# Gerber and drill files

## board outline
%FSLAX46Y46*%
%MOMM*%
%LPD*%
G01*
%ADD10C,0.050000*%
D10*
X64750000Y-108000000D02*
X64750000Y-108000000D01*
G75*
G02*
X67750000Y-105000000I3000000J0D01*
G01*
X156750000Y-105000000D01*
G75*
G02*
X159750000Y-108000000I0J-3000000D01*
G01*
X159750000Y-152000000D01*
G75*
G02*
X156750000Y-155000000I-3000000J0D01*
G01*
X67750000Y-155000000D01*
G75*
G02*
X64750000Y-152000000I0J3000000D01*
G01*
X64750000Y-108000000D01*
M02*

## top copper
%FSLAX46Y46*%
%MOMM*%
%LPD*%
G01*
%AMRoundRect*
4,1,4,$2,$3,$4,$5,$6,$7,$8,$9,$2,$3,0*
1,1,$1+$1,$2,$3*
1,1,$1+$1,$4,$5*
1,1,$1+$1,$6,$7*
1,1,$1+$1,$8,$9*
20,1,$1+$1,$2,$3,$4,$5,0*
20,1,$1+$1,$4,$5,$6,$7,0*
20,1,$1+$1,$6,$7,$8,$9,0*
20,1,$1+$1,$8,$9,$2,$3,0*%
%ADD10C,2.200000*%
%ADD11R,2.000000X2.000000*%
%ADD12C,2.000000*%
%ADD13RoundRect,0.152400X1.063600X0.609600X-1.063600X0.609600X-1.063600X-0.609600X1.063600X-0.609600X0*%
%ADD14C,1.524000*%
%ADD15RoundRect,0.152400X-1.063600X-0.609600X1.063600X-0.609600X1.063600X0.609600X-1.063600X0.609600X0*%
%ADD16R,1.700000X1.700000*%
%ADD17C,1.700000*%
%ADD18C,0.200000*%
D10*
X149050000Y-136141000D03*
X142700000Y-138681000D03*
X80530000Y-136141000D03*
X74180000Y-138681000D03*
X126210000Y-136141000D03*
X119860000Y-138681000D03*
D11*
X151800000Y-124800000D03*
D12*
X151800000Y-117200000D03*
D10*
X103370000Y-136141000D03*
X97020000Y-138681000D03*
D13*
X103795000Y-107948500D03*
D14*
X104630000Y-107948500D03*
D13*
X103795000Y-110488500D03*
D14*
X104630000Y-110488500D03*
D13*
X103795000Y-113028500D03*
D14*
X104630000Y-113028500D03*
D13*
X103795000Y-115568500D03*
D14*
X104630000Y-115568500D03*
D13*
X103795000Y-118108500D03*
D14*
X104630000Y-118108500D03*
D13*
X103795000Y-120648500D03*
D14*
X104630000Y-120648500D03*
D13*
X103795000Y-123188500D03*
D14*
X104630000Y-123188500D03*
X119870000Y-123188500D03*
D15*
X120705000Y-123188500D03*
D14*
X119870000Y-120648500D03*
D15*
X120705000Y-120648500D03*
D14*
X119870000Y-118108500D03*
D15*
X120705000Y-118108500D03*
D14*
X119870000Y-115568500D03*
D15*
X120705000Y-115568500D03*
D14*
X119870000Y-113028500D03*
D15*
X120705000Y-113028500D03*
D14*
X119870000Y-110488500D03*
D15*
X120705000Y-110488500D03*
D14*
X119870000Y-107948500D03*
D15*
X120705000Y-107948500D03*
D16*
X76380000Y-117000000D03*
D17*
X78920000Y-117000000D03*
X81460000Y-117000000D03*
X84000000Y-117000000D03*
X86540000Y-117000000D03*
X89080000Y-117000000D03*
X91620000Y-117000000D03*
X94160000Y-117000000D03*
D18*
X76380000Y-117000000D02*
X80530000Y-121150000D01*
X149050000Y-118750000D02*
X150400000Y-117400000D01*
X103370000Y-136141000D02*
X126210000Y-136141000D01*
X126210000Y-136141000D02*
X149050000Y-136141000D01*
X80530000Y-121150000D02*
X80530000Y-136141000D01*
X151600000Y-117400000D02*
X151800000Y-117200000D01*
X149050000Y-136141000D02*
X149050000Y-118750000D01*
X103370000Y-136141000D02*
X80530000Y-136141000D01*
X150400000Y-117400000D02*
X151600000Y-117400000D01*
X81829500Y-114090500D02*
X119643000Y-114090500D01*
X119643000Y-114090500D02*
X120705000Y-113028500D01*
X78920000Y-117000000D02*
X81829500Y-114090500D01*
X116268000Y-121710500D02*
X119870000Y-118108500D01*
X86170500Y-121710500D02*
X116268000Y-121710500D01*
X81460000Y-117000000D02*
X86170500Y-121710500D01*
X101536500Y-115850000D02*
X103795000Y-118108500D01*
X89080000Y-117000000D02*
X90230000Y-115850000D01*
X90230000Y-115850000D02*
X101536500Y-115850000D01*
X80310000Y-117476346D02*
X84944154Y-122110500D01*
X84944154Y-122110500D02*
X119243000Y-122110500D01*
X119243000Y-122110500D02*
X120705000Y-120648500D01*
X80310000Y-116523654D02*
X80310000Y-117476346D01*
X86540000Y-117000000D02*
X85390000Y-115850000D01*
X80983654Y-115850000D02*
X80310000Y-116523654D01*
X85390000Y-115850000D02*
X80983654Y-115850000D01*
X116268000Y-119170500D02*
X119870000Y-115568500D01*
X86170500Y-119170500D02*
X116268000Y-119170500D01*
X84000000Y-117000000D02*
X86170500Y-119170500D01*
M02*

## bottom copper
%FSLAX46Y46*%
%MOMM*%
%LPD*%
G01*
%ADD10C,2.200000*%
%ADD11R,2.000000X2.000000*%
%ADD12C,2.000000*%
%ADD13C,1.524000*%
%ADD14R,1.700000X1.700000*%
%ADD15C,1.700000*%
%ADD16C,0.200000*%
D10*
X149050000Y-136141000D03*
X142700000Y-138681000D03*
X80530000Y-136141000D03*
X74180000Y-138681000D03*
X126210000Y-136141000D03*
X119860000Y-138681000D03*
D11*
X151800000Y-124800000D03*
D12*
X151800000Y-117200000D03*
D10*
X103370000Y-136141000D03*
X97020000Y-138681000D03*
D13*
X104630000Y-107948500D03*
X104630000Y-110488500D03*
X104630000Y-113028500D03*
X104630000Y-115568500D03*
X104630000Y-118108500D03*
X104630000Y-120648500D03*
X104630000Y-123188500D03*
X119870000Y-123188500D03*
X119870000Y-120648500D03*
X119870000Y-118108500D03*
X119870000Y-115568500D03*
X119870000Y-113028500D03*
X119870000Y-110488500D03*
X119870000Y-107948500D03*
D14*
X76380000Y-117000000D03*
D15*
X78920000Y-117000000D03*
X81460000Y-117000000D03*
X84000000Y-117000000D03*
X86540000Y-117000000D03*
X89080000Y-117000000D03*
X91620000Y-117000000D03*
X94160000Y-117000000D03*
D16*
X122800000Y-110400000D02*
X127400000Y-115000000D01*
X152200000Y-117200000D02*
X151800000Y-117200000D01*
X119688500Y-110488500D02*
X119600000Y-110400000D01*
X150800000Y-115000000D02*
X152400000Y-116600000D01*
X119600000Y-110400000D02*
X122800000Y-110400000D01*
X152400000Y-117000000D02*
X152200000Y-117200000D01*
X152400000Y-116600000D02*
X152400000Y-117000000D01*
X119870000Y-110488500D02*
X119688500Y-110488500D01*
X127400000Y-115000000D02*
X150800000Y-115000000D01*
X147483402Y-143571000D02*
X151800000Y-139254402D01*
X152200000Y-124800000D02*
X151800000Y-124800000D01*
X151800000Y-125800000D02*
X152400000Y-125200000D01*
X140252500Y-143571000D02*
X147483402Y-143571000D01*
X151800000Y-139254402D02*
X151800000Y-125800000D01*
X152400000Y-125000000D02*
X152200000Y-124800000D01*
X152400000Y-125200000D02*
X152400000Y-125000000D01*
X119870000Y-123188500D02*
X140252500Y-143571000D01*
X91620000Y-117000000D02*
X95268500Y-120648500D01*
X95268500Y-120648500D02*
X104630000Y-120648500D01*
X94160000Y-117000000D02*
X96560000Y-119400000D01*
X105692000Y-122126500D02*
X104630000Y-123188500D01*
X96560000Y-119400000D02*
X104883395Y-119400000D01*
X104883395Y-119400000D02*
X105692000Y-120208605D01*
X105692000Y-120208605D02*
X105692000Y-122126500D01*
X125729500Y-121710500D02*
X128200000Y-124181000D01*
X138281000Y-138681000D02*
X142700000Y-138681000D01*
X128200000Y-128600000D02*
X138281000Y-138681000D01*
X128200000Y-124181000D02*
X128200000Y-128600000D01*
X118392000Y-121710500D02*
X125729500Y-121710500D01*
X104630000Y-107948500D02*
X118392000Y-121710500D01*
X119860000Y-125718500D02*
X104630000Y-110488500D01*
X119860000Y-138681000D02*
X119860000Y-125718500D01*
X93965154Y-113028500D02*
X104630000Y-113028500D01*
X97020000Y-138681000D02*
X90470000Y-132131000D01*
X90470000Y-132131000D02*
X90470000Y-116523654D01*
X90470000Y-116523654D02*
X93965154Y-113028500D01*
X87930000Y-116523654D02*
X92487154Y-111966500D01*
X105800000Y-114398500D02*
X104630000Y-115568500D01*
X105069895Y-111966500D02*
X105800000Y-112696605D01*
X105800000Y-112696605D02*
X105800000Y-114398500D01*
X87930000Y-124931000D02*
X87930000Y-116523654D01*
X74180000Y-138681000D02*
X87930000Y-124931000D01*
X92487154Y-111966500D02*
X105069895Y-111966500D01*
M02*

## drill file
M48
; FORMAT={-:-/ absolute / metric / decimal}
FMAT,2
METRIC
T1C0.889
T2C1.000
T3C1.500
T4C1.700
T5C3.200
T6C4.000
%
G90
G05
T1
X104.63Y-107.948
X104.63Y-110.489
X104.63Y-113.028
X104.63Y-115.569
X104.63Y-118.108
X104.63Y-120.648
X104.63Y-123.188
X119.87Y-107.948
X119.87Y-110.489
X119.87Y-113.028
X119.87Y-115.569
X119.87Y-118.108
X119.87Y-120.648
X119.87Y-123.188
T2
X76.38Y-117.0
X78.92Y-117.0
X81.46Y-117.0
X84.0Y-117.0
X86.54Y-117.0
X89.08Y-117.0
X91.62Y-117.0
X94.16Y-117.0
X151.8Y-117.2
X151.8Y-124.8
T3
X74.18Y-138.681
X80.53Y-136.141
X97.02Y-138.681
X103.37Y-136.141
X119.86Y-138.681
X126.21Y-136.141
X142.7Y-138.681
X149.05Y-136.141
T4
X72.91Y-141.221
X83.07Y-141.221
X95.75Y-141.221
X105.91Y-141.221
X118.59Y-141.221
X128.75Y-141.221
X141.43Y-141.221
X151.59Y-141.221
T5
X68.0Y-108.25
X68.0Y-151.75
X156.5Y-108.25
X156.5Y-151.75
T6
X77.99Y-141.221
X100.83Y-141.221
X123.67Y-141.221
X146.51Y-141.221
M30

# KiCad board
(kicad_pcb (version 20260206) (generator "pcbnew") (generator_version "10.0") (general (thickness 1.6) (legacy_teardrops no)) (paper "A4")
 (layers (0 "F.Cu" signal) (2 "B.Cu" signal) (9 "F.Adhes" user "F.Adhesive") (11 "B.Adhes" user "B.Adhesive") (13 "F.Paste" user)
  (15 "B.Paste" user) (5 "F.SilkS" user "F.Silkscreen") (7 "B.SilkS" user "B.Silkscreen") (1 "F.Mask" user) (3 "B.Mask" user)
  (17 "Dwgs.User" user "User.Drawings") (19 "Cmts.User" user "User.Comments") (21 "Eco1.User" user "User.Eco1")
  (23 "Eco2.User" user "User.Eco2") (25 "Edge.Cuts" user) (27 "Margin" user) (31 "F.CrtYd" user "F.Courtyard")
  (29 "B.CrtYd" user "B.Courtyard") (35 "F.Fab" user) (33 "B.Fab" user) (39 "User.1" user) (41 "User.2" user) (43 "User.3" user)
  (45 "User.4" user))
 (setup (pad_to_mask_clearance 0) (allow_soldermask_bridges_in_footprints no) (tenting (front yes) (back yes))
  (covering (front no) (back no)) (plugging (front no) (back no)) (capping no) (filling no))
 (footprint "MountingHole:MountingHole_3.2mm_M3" (layer "F.Cu") (at 156.5 108.25 90)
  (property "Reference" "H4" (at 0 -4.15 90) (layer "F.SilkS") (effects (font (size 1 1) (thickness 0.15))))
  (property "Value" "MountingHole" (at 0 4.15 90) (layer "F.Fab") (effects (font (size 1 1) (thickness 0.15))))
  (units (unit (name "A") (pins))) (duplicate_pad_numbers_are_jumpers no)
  (pad "" np_thru_hole circle (at 0 0 90) (size 3.2 3.2) (drill 3.2) (layers "*.Cu" "*.Mask")))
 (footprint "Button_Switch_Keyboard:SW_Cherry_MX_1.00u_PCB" (layer "F.Cu") (at 149.05 136.141)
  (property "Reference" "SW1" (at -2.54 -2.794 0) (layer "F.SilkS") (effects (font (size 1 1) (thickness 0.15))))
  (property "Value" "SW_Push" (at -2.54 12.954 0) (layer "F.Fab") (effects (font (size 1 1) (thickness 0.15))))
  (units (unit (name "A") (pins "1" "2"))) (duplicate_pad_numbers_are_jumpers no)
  (pad "" np_thru_hole circle (at -7.62 5.08) (size 1.7 1.7) (drill 1.7) (layers "*.Cu" "*.Mask"))
  (pad "" np_thru_hole circle (at -2.54 5.08) (size 4 4) (drill 4) (layers "*.Cu" "*.Mask"))
  (pad "" np_thru_hole circle (at 2.54 5.08) (size 1.7 1.7) (drill 1.7) (layers "*.Cu" "*.Mask"))
  (pad "1" thru_hole circle (at 0 0) (size 2.2 2.2) (drill 1.5) (layers "*.Cu" "*.Mask") (remove_unused_layers no) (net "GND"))
  (pad "2" thru_hole circle (at -6.35 2.54) (size 2.2 2.2) (drill 1.5) (layers "*.Cu" "*.Mask") (remove_unused_layers no)
   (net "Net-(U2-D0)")))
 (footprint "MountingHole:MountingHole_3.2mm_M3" (layer "F.Cu") (at 156.5 151.75 90)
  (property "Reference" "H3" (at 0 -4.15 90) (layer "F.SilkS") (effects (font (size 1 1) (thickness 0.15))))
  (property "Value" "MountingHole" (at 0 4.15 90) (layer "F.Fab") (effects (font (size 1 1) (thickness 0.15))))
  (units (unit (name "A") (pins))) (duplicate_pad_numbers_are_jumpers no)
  (pad "" np_thru_hole circle (at 0 0 90) (size 3.2 3.2) (drill 3.2) (layers "*.Cu" "*.Mask")))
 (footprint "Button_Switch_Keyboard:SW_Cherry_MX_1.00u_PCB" (layer "F.Cu") (at 80.53 136.141)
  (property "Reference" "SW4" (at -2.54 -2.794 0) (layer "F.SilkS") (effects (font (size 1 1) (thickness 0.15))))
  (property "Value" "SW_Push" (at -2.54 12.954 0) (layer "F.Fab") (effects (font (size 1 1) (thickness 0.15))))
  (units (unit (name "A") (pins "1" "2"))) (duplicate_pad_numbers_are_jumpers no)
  (pad "" np_thru_hole circle (at -7.62 5.08) (size 1.7 1.7) (drill 1.7) (layers "*.Cu" "*.Mask"))
  (pad "" np_thru_hole circle (at -2.54 5.08) (size 4 4) (drill 4) (layers "*.Cu" "*.Mask"))
  (pad "" np_thru_hole circle (at 2.54 5.08) (size 1.7 1.7) (drill 1.7) (layers "*.Cu" "*.Mask"))
  (pad "1" thru_hole circle (at 0 0) (size 2.2 2.2) (drill 1.5) (layers "*.Cu" "*.Mask") (remove_unused_layers no) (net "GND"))
  (pad "2" thru_hole circle (at -6.35 2.54) (size 2.2 2.2) (drill 1.5) (layers "*.Cu" "*.Mask") (remove_unused_layers no)
   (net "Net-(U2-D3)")))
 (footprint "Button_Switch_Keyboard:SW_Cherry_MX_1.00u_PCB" (layer "F.Cu") (at 126.21 136.141)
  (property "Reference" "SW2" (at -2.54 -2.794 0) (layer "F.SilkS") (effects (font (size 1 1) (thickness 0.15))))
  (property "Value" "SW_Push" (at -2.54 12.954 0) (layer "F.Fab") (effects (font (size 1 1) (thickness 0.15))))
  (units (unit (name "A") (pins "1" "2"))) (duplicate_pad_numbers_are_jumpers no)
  (pad "" np_thru_hole circle (at -7.62 5.08) (size 1.7 1.7) (drill 1.7) (layers "*.Cu" "*.Mask"))
  (pad "" np_thru_hole circle (at -2.54 5.08) (size 4 4) (drill 4) (layers "*.Cu" "*.Mask"))
  (pad "" np_thru_hole circle (at 2.54 5.08) (size 1.7 1.7) (drill 1.7) (layers "*.Cu" "*.Mask"))
  (pad "1" thru_hole circle (at 0 0) (size 2.2 2.2) (drill 1.5) (layers "*.Cu" "*.Mask") (remove_unused_layers no) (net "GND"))
  (pad "2" thru_hole circle (at -6.35 2.54) (size 2.2 2.2) (drill 1.5) (layers "*.Cu" "*.Mask") (remove_unused_layers no)
   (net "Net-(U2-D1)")))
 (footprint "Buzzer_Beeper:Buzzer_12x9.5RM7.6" (layer "F.Cu") (at 151.8 124.8 90)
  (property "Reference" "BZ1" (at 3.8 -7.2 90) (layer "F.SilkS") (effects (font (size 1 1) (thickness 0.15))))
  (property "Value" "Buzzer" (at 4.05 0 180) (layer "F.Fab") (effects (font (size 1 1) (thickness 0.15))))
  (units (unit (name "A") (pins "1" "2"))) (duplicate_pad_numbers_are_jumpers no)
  (pad "1" thru_hole rect (at 0 0 90) (size 2 2) (drill 1) (layers "*.Cu" "*.Mask") (remove_unused_layers no) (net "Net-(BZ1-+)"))
  (pad "2" thru_hole circle (at 7.6 0 90) (size 2 2) (drill 1) (layers "*.Cu" "*.Mask") (remove_unused_layers no) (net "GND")))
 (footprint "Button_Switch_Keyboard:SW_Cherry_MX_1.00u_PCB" (layer "F.Cu") (at 103.37 136.141)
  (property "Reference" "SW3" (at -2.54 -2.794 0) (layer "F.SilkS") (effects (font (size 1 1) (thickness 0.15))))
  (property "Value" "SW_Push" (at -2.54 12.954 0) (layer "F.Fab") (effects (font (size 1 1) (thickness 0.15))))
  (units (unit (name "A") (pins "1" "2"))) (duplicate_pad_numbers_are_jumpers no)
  (pad "" np_thru_hole circle (at -7.62 5.08) (size 1.7 1.7) (drill 1.7) (layers "*.Cu" "*.Mask"))
  (pad "" np_thru_hole circle (at -2.54 5.08) (size 4 4) (drill 4) (layers "*.Cu" "*.Mask"))
  (pad "" np_thru_hole circle (at 2.54 5.08) (size 1.7 1.7) (drill 1.7) (layers "*.Cu" "*.Mask"))
  (pad "1" thru_hole circle (at 0 0) (size 2.2 2.2) (drill 1.5) (layers "*.Cu" "*.Mask") (remove_unused_layers no) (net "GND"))
  (pad "2" thru_hole circle (at -6.35 2.54) (size 2.2 2.2) (drill 1.5) (layers "*.Cu" "*.Mask") (remove_unused_layers no)
   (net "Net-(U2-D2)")))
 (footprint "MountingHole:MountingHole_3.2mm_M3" (layer "F.Cu") (at 68 108.25 90)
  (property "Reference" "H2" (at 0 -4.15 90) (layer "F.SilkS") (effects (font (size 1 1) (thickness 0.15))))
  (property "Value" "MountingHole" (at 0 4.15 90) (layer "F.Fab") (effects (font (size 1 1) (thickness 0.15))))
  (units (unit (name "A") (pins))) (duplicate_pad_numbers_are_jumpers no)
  (pad "" np_thru_hole circle (at 0 0 90) (size 3.2 3.2) (drill 3.2) (layers "*.Cu" "*.Mask")))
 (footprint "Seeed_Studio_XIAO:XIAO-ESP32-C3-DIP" (layer "F.Cu") (at 112.25 115.5685 90)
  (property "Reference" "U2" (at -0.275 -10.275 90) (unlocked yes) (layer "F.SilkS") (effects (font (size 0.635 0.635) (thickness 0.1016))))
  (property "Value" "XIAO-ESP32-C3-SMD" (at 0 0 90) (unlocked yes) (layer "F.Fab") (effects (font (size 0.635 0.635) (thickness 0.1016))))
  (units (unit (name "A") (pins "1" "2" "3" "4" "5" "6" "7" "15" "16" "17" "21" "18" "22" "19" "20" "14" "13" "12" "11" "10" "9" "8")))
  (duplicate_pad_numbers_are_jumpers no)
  (pad "1" smd roundrect (at 7.62 -8.455 180) (size 2.432 1.524) (layers "F.Cu" "F.Mask") (roundrect_rratio 0.1) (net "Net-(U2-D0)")
   (thermal_bridge_angle 45))
  (pad "1" thru_hole circle (at 7.62 -7.62 180) (size 1.524 1.524) (drill 0.889) (layers "*.Cu" "*.Mask") (remove_unused_layers no)
   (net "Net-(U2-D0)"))
  (pad "2" smd roundrect (at 5.08 -8.455 180) (size 2.432 1.524) (layers "F.Cu" "F.Mask") (roundrect_rratio 0.1) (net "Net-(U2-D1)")
   (thermal_bridge_angle 45))
  (pad "2" thru_hole circle (at 5.08 -7.62 180) (size 1.524 1.524) (drill 0.889) (layers "*.Cu" "*.Mask") (remove_unused_layers no)
   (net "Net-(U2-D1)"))
  (pad "3" smd roundrect (at 2.54 -8.455 180) (size 2.432 1.524) (layers "F.Cu" "F.Mask") (roundrect_rratio 0.1) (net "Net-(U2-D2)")
   (thermal_bridge_angle 45))
  (pad "3" thru_hole circle (at 2.54 -7.62 180) (size 1.524 1.524) (drill 0.889) (layers "*.Cu" "*.Mask") (remove_unused_layers no)
   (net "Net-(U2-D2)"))
  (pad "4" smd roundrect (at 0 -8.455 180) (size 2.432 1.524) (layers "F.Cu" "F.Mask") (roundrect_rratio 0.1) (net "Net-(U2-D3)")
   (thermal_bridge_angle 45))
  (pad "4" thru_hole circle (at 0 -7.62 180) (size 1.524 1.524) (drill 0.889) (layers "*.Cu" "*.Mask") (remove_unused_layers no)
   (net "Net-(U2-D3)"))
  (pad "5" smd roundrect (at -2.54 -8.455 180) (size 2.432 1.524) (layers "F.Cu" "F.Mask") (roundrect_rratio 0.1) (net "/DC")
   (thermal_bridge_angle 45))
  (pad "5" thru_hole circle (at -2.54 -7.62 180) (size 1.524 1.524) (drill 0.889) (layers "*.Cu" "*.Mask") (remove_unused_layers no)
   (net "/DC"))
  (pad "6" smd roundrect (at -5.08 -8.455 180) (size 2.432 1.524) (layers "F.Cu" "F.Mask") (roundrect_rratio 0.1) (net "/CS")
   (thermal_bridge_angle 45))
  (pad "6" thru_hole circle (at -5.08 -7.62 180) (size 1.524 1.524) (drill 0.889) (layers "*.Cu" "*.Mask") (remove_unused_layers no)
   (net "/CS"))
  (pad "7" smd roundrect (at -7.62 -8.455 180) (size 2.432 1.524) (layers "F.Cu" "F.Mask") (roundrect_rratio 0.1) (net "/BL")
   (thermal_bridge_angle 45))
  (pad "7" thru_hole circle (at -7.62 -7.62 180) (size 1.524 1.524) (drill 0.889) (layers "*.Cu" "*.Mask") (remove_unused_layers no)
   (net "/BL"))
  (pad "8" thru_hole circle (at -7.62 7.62) (size 1.524 1.524) (drill 0.889) (layers "*.Cu" "*.Mask") (remove_unused_layers no)
   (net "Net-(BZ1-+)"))
  (pad "8" smd roundrect (at -7.62 8.455) (size 2.432 1.524) (layers "F.Cu" "F.Mask") (roundrect_rratio 0.1) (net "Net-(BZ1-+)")
   (thermal_bridge_angle 45))
  (pad "9" thru_hole circle (at -5.08 7.62) (size 1.524 1.524) (drill 0.889) (layers "*.Cu" "*.Mask") (remove_unused_layers no) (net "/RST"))
  (pad "9" smd roundrect (at -5.08 8.455) (size 2.432 1.524) (layers "F.Cu" "F.Mask") (roundrect_rratio 0.1) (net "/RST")
   (thermal_bridge_angle 45))
  (pad "10" thru_hole circle (at -2.54 7.62) (size 1.524 1.524) (drill 0.889) (layers "*.Cu" "*.Mask") (remove_unused_layers no)
   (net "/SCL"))
  (pad "10" smd roundrect (at -2.54 8.455) (size 2.432 1.524) (layers "F.Cu" "F.Mask") (roundrect_rratio 0.1) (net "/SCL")
   (thermal_bridge_angle 45))
  (pad "11" thru_hole circle (at 0 7.62) (size 1.524 1.524) (drill 0.889) (layers "*.Cu" "*.Mask") (remove_unused_layers no) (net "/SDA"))
  (pad "11" smd roundrect (at 0 8.455) (size 2.432 1.524) (layers "F.Cu" "F.Mask") (roundrect_rratio 0.1) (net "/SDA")
   (thermal_bridge_angle 45))
  (pad "12" thru_hole circle (at 2.54 7.62) (size 1.524 1.524) (drill 0.889) (layers "*.Cu" "*.Mask") (remove_unused_layers no)
   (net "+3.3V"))
  (pad "12" smd roundrect (at 2.54 8.455) (size 2.432 1.524) (layers "F.Cu" "F.Mask") (roundrect_rratio 0.1) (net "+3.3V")
   (thermal_bridge_angle 45))
  (pad "13" thru_hole circle (at 5.08 7.62) (size 1.524 1.524) (drill 0.889) (layers "*.Cu" "*.Mask") (remove_unused_layers no) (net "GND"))
  (pad "13" smd roundrect (at 5.08 8.455) (size 2.432 1.524) (layers "F.Cu" "F.Mask") (roundrect_rratio 0.1) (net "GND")
   (thermal_bridge_angle 45))
  (pad "14" thru_hole circle (at 7.62 7.62) (size 1.524 1.524) (drill 0.889) (layers "*.Cu" "*.Mask") (remove_unused_layers no)
   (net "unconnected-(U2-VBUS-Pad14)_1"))
  (pad "14" smd roundrect (at 7.62 8.455) (size 2.432 1.524) (layers "F.Cu" "F.Mask") (roundrect_rratio 0.1)
   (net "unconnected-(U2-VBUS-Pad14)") (thermal_bridge_angle 45)))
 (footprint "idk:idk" (layer "F.Cu") (at 135.6 121.6)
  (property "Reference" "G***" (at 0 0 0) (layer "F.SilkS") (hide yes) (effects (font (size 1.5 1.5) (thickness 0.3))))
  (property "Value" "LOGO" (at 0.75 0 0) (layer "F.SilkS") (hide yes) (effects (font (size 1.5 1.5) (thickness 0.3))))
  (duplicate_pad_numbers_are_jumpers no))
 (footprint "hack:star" (layer "F.Cu") (at 136.4 110.8)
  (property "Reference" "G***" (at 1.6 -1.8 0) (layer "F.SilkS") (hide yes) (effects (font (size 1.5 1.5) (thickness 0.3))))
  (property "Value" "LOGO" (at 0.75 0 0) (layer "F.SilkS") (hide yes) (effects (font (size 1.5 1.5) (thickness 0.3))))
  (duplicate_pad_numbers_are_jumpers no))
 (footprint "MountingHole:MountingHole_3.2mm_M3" (layer "F.Cu") (at 68 151.75 90)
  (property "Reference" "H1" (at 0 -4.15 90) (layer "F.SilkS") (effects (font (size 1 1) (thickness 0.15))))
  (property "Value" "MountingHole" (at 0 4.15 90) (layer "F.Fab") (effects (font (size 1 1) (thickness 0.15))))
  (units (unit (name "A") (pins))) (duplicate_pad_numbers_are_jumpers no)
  (pad "" np_thru_hole circle (at 0 0 90) (size 3.2 3.2) (drill 3.2) (layers "*.Cu" "*.Mask")))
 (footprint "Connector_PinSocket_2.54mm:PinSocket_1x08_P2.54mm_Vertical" (layer "B.Cu") (at 76.38 117 -90)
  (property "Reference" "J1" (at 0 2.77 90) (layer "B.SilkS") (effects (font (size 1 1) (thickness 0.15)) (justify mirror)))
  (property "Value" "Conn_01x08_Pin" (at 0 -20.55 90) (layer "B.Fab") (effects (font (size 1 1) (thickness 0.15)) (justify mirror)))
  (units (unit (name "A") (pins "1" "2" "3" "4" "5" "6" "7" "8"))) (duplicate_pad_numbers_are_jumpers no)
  (pad "1" thru_hole rect (at 0 0 270) (size 1.7 1.7) (drill 1) (layers "*.Cu" "*.Mask") (remove_unused_layers no) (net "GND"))
  (pad "2" thru_hole circle (at 0 -2.54 270) (size 1.7 1.7) (drill 1) (layers "*.Cu" "*.Mask") (remove_unused_layers no) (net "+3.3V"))
  (pad "3" thru_hole circle (at 0 -5.08 270) (size 1.7 1.7) (drill 1) (layers "*.Cu" "*.Mask") (remove_unused_layers no) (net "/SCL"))
  (pad "4" thru_hole circle (at 0 -7.62 270) (size 1.7 1.7) (drill 1) (layers "*.Cu" "*.Mask") (remove_unused_layers no) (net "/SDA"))
  (pad "5" thru_hole circle (at 0 -10.16 270) (size 1.7 1.7) (drill 1) (layers "*.Cu" "*.Mask") (remove_unused_layers no) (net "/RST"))
  (pad "6" thru_hole circle (at 0 -12.7 270) (size 1.7 1.7) (drill 1) (layers "*.Cu" "*.Mask") (remove_unused_layers no) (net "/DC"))
  (pad "7" thru_hole circle (at 0 -15.24 270) (size 1.7 1.7) (drill 1) (layers "*.Cu" "*.Mask") (remove_unused_layers no) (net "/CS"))
  (pad "8" thru_hole circle (at 0 -17.78 270) (size 1.7 1.7) (drill 1) (layers "*.Cu" "*.Mask") (remove_unused_layers no) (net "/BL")))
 (gr_rect (start 64.75 105) (end 159.75 155) (radius 3) (stroke (width 0.05) (type default)) (fill no) (layer "Edge.Cuts"))
 (segment (start 76.38 117) (end 80.53 121.15) (width 0.2) (layer "F.Cu") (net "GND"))
 (segment (start 149.05 118.75) (end 150.4 117.4) (width 0.2) (layer "F.Cu") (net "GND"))
 (segment (start 103.37 136.141) (end 126.21 136.141) (width 0.2) (layer "F.Cu") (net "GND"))
 (segment (start 126.21 136.141) (end 149.05 136.141) (width 0.2) (layer "F.Cu") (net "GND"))
 (segment (start 80.53 121.15) (end 80.53 136.141) (width 0.2) (layer "F.Cu") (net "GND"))
 (segment (start 151.6 117.4) (end 151.8 117.2) (width 0.2) (layer "F.Cu") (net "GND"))
 (segment (start 149.05 136.141) (end 149.05 118.75) (width 0.2) (layer "F.Cu") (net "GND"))
 (segment (start 103.37 136.141) (end 80.53 136.141) (width 0.2) (layer "F.Cu") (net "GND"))
 (segment (start 150.4 117.4) (end 151.6 117.4) (width 0.2) (layer "F.Cu") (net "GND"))
 (segment (start 122.8 110.4) (end 127.4 115) (width 0.2) (layer "B.Cu") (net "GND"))
 (segment (start 152.2 117.2) (end 151.8 117.2) (width 0.2) (layer "B.Cu") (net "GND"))
 (segment (start 119.6885 110.4885) (end 119.6 110.4) (width 0.2) (layer "B.Cu") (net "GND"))
 (segment (start 150.8 115) (end 152.4 116.6) (width 0.2) (layer "B.Cu") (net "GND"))
 (segment (start 119.6 110.4) (end 122.8 110.4) (width 0.2) (layer "B.Cu") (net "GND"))
 (segment (start 152.4 117) (end 152.2 117.2) (width 0.2) (layer "B.Cu") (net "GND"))
 (segment (start 152.4 116.6) (end 152.4 117) (width 0.2) (layer "B.Cu") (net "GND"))
 (segment (start 119.87 110.4885) (end 119.6885 110.4885) (width 0.2) (layer "B.Cu") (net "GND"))
 (segment (start 127.4 115) (end 150.8 115) (width 0.2) (layer "B.Cu") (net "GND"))
 (segment (start 147.483402 143.571) (end 151.8 139.254402) (width 0.2) (layer "B.Cu") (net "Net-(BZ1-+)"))
 (segment (start 152.2 124.8) (end 151.8 124.8) (width 0.2) (layer "B.Cu") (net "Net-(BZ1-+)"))
 (segment (start 151.8 125.8) (end 152.4 125.2) (width 0.2) (layer "B.Cu") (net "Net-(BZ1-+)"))
 (segment (start 140.2525 143.571) (end 147.483402 143.571) (width 0.2) (layer "B.Cu") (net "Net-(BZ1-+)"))
 (segment (start 151.8 139.254402) (end 151.8 125.8) (width 0.2) (layer "B.Cu") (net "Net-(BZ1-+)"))
 (segment (start 152.4 125) (end 152.2 124.8) (width 0.2) (layer "B.Cu") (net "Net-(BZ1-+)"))
 (segment (start 152.4 125.2) (end 152.4 125) (width 0.2) (layer "B.Cu") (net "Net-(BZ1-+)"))
 (segment (start 119.87 123.1885) (end 140.2525 143.571) (width 0.2) (layer "B.Cu") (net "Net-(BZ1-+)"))
 (segment (start 91.62 117) (end 95.2685 120.6485) (width 0.2) (layer "B.Cu") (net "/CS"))
 (segment (start 95.2685 120.6485) (end 104.63 120.6485) (width 0.2) (layer "B.Cu") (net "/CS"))
 (segment (start 81.8295 114.0905) (end 119.643 114.0905) (width 0.2) (layer "F.Cu") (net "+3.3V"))
 (segment (start 119.643 114.0905) (end 120.705 113.0285) (width 0.2) (layer "F.Cu") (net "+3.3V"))
 (segment (start 78.92 117) (end 81.8295 114.0905) (width 0.2) (layer "F.Cu") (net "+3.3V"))
 (segment (start 116.268 121.7105) (end 119.87 118.1085) (width 0.2) (layer "F.Cu") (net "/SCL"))
 (segment (start 86.1705 121.7105) (end 116.268 121.7105) (width 0.2) (layer "F.Cu") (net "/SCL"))
 (segment (start 81.46 117) (end 86.1705 121.7105) (width 0.2) (layer "F.Cu") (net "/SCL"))
 (segment (start 101.5365 115.85) (end 103.795 118.1085) (width 0.2) (layer "F.Cu") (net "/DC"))
 (segment (start 89.08 117) (end 90.23 115.85) (width 0.2) (layer "F.Cu") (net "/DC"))
 (segment (start 90.23 115.85) (end 101.5365 115.85) (width 0.2) (layer "F.Cu") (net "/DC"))
 (segment (start 80.31 117.476346) (end 84.944154 122.1105) (width 0.2) (layer "F.Cu") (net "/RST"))
 (segment (start 84.944154 122.1105) (end 119.243 122.1105) (width 0.2) (layer "F.Cu") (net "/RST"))
 (segment (start 119.243 122.1105) (end 120.705 120.6485) (width 0.2) (layer "F.Cu") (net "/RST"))
 (segment (start 80.31 116.523654) (end 80.31 117.476346) (width 0.2) (layer "F.Cu") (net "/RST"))
 (segment (start 86.54 117) (end 85.39 115.85) (width 0.2) (layer "F.Cu") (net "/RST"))
 (segment (start 80.983654 115.85) (end 80.31 116.523654) (width 0.2) (layer "F.Cu") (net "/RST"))
 (segment (start 85.39 115.85) (end 80.983654 115.85) (width 0.2) (layer "F.Cu") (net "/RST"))
 (segment (start 116.268 119.1705) (end 119.87 115.5685) (width 0.2) (layer "F.Cu") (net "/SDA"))
 (segment (start 86.1705 119.1705) (end 116.268 119.1705) (width 0.2) (layer "F.Cu") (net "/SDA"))
 (segment (start 84 117) (end 86.1705 119.1705) (width 0.2) (layer "F.Cu") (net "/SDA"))
 (segment (start 94.16 117) (end 96.56 119.4) (width 0.2) (layer "B.Cu") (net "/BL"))
 (segment (start 105.692 122.1265) (end 104.63 123.1885) (width 0.2) (layer "B.Cu") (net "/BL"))
 (segment (start 96.56 119.4) (end 104.883395 119.4) (width 0.2) (layer "B.Cu") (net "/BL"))
 (segment (start 104.883395 119.4) (end 105.692 120.208605) (width 0.2) (layer "B.Cu") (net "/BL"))
 (segment (start 105.692 120.208605) (end 105.692 122.1265) (width 0.2) (layer "B.Cu") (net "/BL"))
 (segment (start 125.7295 121.7105) (end 128.2 124.181) (width 0.2) (layer "B.Cu") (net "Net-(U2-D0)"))
 (segment (start 138.281 138.681) (end 142.7 138.681) (width 0.2) (layer "B.Cu") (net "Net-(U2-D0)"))
 (segment (start 128.2 128.6) (end 138.281 138.681) (width 0.2) (layer "B.Cu") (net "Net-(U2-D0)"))
 (segment (start 128.2 124.181) (end 128.2 128.6) (width 0.2) (layer "B.Cu") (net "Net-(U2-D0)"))
 (segment (start 118.392 121.7105) (end 125.7295 121.7105) (width 0.2) (layer "B.Cu") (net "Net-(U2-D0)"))
 (segment (start 104.63 107.9485) (end 118.392 121.7105) (width 0.2) (layer "B.Cu") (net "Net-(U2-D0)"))
 (segment (start 119.86 125.7185) (end 104.63 110.4885) (width 0.2) (layer "B.Cu") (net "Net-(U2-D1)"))
 (segment (start 119.86 138.681) (end 119.86 125.7185) (width 0.2) (layer "B.Cu") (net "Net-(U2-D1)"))
 (segment (start 93.965154 113.0285) (end 104.63 113.0285) (width 0.2) (layer "B.Cu") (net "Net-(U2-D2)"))
 (segment (start 97.02 138.681) (end 90.47 132.131) (width 0.2) (layer "B.Cu") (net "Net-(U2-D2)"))
 (segment (start 90.47 132.131) (end 90.47 116.523654) (width 0.2) (layer "B.Cu") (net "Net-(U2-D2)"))
 (segment (start 90.47 116.523654) (end 93.965154 113.0285) (width 0.2) (layer "B.Cu") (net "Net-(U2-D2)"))
 (segment (start 87.93 116.523654) (end 92.487154 111.9665) (width 0.2) (layer "B.Cu") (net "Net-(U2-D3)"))
 (segment (start 105.8 114.3985) (end 104.63 115.5685) (width 0.2) (layer "B.Cu") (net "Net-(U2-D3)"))
 (segment (start 105.069895 111.9665) (end 105.8 112.696605) (width 0.2) (layer "B.Cu") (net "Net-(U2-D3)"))
 (segment (start 105.8 112.696605) (end 105.8 114.3985) (width 0.2) (layer "B.Cu") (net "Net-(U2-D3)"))
 (segment (start 87.93 124.931) (end 87.93 116.523654) (width 0.2) (layer "B.Cu") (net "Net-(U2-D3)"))
 (segment (start 74.18 138.681) (end 87.93 124.931) (width 0.2) (layer "B.Cu") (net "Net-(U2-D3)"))
 (segment (start 92.487154 111.9665) (end 105.069895 111.9665) (width 0.2) (layer "B.Cu") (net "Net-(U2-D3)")))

